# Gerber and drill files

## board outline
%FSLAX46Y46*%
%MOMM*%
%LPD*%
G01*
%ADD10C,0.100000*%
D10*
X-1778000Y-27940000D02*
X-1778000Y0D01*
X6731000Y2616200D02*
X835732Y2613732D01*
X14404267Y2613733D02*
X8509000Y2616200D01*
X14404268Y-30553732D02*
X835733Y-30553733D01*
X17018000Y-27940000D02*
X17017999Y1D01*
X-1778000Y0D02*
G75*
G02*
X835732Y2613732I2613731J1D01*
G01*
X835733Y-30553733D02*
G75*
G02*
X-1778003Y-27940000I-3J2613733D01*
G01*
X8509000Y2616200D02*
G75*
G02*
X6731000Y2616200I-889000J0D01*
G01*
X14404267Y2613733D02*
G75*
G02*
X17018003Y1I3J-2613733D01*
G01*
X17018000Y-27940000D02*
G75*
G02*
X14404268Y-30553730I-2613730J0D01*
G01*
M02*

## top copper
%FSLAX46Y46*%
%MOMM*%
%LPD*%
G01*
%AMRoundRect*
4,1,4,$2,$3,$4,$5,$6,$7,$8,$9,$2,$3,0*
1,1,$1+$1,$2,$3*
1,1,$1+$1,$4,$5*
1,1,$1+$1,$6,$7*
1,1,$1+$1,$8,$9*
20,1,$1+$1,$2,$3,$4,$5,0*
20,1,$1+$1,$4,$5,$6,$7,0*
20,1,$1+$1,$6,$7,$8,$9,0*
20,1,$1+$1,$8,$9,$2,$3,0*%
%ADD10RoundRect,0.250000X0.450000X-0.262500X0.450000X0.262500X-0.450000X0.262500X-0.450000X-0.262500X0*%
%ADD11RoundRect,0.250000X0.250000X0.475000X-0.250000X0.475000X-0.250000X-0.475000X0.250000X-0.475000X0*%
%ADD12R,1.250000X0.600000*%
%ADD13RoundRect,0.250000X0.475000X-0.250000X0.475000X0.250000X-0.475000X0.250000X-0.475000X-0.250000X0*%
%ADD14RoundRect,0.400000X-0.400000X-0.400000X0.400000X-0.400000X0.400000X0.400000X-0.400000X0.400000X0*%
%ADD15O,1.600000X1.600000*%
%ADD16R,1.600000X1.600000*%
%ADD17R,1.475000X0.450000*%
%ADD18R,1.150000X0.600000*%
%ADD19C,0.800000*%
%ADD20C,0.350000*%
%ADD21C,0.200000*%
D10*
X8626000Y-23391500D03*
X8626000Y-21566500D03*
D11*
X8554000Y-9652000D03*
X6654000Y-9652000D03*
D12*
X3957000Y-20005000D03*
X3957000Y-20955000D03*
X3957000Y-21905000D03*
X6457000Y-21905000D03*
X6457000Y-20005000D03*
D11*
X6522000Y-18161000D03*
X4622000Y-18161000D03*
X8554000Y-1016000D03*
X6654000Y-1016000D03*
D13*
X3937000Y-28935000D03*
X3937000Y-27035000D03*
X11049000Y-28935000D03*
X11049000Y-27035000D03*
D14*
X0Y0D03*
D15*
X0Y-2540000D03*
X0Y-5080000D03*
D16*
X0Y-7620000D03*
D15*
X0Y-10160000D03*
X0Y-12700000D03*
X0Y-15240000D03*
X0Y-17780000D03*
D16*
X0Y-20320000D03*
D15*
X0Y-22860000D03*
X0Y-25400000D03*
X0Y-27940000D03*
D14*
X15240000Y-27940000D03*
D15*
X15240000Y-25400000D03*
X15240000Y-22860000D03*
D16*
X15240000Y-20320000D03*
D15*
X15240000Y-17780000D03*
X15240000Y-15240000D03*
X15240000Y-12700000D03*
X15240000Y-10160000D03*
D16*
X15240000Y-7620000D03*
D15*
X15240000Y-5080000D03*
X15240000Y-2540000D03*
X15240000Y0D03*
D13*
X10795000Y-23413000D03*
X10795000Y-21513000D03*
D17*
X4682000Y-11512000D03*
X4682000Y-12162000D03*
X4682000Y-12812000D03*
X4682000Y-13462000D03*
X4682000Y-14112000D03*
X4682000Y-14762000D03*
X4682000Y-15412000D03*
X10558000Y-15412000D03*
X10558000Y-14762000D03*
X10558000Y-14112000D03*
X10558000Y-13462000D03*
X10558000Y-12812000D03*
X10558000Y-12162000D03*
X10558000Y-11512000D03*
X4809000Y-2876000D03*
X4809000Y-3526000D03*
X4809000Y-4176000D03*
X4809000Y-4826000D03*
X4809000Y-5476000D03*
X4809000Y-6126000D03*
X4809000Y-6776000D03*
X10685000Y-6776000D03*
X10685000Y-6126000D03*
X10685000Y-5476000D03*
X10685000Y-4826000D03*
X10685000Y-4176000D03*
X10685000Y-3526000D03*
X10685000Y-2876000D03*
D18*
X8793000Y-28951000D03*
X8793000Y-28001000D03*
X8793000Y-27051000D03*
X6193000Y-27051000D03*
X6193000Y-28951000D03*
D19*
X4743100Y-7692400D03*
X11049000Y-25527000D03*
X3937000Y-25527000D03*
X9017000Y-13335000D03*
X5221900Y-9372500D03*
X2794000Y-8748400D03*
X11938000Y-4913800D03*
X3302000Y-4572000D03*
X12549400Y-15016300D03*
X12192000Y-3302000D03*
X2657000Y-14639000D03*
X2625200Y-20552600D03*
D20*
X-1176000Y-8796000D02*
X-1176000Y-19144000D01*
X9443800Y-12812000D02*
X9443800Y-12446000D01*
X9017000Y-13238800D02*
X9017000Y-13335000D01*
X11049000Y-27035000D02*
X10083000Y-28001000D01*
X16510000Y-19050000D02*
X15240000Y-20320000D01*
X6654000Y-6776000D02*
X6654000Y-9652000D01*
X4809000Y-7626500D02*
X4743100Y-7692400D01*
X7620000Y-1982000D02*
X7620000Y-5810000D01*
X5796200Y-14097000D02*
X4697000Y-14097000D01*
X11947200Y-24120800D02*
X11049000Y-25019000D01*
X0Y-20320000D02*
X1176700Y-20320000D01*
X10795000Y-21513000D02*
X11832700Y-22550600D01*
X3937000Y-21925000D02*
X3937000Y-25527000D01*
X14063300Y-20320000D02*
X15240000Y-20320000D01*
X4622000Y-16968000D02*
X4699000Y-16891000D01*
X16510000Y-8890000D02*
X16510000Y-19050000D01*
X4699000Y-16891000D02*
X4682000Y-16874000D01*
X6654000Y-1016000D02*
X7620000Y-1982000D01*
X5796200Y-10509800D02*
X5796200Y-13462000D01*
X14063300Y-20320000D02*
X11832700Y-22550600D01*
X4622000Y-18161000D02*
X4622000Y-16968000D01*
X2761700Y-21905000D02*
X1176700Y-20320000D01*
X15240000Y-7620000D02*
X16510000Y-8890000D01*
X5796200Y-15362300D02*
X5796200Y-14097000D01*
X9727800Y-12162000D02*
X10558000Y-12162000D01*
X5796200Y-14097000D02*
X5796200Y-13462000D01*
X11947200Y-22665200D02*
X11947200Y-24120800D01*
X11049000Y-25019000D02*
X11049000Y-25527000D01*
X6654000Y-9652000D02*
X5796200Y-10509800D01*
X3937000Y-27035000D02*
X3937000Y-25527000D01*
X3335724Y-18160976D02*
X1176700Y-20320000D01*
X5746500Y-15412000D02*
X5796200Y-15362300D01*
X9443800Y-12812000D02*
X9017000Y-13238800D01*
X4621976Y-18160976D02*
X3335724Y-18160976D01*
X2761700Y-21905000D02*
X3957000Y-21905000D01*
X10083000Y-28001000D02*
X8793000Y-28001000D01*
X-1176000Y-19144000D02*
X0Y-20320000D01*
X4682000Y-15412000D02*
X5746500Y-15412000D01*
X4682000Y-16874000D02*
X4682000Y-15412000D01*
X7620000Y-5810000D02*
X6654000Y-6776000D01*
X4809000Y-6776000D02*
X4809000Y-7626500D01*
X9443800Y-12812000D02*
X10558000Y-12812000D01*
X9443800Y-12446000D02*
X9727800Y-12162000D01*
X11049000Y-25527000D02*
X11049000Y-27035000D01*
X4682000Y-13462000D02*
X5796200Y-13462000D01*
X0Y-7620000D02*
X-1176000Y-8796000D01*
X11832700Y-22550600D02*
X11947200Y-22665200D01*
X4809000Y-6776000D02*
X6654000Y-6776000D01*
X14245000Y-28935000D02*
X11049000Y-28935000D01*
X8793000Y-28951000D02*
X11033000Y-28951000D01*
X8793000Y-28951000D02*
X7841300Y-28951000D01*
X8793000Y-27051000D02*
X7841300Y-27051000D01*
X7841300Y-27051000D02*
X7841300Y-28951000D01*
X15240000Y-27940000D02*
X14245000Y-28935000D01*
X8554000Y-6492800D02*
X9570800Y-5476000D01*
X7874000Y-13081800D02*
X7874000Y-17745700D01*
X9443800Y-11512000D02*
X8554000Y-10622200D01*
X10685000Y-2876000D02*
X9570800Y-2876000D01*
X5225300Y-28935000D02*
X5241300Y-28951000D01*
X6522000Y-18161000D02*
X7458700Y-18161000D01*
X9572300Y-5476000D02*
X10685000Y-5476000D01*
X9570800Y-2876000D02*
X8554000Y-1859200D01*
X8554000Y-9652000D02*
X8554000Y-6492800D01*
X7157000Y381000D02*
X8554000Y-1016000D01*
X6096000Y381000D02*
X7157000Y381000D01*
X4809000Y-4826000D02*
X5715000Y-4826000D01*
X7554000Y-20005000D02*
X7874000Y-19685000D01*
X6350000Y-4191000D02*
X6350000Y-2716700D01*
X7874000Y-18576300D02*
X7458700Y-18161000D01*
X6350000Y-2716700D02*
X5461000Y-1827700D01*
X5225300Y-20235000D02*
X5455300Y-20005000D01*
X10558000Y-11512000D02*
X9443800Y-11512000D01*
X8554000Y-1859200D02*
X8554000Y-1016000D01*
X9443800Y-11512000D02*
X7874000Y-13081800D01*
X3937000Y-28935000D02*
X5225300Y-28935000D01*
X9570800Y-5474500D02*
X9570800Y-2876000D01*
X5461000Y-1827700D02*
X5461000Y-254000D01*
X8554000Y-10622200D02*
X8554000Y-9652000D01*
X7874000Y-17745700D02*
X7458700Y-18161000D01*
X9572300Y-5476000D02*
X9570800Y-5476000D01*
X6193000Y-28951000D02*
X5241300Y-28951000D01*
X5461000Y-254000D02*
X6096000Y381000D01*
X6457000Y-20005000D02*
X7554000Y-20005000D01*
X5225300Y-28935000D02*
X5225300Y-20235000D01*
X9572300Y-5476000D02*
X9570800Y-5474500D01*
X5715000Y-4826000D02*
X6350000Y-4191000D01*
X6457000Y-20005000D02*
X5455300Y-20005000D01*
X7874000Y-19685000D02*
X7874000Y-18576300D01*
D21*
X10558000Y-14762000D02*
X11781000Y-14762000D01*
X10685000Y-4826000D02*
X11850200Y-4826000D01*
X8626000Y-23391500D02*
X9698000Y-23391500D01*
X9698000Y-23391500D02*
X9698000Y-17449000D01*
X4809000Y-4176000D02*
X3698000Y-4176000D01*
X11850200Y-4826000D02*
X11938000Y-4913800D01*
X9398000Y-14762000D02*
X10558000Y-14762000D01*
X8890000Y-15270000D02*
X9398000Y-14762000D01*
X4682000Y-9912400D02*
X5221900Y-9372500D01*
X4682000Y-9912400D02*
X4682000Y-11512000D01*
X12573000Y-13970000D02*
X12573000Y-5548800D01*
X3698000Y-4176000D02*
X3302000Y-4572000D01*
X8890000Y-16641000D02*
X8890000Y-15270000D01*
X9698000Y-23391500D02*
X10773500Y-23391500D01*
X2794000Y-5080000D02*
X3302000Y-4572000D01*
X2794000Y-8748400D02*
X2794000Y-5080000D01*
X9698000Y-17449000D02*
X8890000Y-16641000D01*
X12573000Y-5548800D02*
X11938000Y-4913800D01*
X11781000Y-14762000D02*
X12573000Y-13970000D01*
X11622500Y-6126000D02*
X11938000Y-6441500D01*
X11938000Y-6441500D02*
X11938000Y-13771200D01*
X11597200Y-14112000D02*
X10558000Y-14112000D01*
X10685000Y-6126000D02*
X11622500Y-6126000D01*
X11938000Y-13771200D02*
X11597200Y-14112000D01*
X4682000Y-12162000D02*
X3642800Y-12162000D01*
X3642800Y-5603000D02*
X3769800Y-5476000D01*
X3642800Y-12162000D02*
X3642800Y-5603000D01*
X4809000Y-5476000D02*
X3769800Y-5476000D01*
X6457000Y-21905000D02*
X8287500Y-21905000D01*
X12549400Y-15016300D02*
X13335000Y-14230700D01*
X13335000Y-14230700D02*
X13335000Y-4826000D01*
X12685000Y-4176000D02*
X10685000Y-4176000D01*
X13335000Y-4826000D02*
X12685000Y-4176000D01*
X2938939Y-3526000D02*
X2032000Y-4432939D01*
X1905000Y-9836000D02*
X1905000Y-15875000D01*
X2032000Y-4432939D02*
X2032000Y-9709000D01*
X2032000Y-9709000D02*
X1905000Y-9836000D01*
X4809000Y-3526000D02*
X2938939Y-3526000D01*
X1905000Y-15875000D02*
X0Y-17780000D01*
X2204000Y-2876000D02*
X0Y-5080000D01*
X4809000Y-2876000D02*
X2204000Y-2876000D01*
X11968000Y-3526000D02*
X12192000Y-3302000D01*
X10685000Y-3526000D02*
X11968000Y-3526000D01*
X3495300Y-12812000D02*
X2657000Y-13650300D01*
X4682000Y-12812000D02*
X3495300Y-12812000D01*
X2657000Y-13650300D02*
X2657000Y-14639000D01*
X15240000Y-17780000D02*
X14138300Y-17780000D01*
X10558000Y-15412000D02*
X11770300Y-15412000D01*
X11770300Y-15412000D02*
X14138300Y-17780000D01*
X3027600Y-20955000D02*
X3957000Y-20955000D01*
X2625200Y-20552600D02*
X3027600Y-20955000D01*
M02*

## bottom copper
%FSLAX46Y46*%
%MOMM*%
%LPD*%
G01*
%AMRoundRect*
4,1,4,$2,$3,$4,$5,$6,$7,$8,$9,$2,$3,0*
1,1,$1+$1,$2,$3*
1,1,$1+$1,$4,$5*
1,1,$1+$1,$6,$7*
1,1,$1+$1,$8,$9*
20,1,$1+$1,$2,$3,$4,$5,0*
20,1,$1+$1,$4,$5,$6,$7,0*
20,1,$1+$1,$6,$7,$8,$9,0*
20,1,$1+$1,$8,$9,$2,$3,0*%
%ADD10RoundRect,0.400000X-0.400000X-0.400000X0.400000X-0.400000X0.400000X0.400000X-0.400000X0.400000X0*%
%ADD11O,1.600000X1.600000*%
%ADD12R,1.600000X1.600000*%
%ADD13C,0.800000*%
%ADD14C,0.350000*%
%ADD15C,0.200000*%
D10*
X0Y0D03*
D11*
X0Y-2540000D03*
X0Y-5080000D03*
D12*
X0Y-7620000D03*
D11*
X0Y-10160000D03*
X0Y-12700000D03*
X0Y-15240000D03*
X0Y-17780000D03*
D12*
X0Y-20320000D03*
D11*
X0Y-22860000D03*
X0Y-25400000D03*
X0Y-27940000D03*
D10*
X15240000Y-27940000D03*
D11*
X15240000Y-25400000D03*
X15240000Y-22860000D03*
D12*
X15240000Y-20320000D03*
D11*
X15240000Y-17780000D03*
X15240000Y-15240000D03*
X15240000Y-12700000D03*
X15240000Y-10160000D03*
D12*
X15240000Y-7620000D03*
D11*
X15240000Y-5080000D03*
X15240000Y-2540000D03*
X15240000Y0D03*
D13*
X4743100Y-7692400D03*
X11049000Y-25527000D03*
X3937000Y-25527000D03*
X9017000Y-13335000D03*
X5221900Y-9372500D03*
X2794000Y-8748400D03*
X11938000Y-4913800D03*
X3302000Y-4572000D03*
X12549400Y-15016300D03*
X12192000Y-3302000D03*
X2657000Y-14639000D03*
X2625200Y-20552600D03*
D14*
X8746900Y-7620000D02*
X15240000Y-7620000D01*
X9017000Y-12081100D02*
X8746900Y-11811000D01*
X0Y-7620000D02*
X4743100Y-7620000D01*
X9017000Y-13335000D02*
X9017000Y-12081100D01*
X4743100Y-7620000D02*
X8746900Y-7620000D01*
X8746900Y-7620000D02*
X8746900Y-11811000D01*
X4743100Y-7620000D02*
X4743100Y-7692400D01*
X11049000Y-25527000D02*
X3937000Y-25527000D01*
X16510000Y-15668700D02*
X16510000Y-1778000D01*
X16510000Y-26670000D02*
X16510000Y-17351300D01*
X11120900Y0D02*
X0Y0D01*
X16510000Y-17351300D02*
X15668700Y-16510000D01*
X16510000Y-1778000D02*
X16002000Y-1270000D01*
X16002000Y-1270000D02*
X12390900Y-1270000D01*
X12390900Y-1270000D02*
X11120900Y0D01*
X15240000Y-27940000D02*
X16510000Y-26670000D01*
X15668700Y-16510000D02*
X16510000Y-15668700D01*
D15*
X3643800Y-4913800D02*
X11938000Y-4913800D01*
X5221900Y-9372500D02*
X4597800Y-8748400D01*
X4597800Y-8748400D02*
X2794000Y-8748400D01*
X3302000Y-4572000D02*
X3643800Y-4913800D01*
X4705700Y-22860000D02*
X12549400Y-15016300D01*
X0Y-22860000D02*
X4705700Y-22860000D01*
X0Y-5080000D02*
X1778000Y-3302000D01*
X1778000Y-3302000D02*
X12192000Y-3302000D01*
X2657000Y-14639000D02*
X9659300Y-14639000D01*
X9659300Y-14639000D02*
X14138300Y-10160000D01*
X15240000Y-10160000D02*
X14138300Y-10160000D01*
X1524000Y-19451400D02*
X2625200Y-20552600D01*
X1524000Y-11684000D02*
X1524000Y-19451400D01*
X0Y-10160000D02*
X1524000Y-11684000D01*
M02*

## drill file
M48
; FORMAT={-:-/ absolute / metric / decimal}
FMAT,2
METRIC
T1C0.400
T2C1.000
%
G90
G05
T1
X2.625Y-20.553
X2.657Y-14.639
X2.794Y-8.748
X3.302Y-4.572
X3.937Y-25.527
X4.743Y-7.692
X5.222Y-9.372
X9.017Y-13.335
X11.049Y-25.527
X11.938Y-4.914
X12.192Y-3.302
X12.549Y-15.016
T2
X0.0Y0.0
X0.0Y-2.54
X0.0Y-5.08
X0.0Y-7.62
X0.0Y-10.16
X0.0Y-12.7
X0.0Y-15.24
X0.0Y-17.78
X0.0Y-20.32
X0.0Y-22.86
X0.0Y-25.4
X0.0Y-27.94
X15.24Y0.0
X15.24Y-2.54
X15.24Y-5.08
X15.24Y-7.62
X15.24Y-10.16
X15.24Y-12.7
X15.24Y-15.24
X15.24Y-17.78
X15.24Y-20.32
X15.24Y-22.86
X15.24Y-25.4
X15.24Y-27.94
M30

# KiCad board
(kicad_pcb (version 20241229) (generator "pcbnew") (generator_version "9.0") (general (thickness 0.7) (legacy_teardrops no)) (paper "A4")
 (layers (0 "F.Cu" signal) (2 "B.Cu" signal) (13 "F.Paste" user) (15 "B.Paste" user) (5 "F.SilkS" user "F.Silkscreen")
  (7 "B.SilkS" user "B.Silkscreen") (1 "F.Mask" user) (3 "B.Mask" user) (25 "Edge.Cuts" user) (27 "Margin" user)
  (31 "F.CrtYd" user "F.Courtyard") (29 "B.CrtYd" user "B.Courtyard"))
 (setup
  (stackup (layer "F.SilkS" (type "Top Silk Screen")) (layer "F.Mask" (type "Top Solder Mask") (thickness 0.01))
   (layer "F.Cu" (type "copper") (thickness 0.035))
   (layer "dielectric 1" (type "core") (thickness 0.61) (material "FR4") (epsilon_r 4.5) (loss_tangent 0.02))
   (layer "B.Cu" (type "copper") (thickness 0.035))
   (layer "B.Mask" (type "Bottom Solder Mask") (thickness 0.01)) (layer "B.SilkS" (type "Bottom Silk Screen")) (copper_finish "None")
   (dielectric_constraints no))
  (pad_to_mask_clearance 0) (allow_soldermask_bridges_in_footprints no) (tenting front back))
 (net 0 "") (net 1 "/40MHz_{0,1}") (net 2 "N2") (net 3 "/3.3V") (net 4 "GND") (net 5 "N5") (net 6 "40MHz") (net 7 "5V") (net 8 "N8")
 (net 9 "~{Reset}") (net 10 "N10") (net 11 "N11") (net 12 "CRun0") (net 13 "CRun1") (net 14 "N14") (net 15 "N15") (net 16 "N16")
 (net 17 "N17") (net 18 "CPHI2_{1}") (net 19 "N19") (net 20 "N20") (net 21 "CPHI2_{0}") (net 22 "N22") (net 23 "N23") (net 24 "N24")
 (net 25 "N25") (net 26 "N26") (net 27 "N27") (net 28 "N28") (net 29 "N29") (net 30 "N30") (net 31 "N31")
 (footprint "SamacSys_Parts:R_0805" (layer "F.Cu") (at 8.636 22.479)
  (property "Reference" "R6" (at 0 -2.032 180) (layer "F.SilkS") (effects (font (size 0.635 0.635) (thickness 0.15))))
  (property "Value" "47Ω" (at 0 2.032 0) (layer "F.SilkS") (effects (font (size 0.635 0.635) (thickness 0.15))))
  (pad "1" smd roundrect (at -0.01 0.9125 90) (size 1.025 1.4) (layers "F.Cu" "F.Mask" "F.Paste") (roundrect_rratio 0.243902)
   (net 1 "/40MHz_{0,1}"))
  (pad "2" smd roundrect (at -0.01 -0.9125 90) (size 1.025 1.4) (layers "F.Cu" "F.Mask" "F.Paste") (roundrect_rratio 0.243902) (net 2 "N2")))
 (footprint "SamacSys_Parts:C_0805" (layer "F.Cu") (at 7.62 9.652 90)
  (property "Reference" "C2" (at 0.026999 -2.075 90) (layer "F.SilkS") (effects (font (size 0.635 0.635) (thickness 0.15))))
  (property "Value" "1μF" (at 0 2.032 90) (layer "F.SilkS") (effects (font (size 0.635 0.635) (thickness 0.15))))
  (pad "1" smd roundrect (at 0 0.934 180) (size 1 1.45) (layers "F.Cu" "F.Mask" "F.Paste") (roundrect_rratio 0.25) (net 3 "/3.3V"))
  (pad "2" smd roundrect (at 0 -0.966 180) (size 1 1.45) (layers "F.Cu" "F.Mask" "F.Paste") (roundrect_rratio 0.25) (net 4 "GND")))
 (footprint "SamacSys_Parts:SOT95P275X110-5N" (layer "F.Cu") (at 5.207 20.955)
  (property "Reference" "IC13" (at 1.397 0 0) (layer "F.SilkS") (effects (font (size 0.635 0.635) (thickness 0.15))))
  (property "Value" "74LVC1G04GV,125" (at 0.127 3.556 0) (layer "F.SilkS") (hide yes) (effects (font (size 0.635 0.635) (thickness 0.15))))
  (pad "1" smd rect (at -1.25 -0.95 90) (size 0.6 1.25) (layers "F.Cu" "F.Mask" "F.Paste") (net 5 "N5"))
  (pad "2" smd rect (at -1.25 0 90) (size 0.6 1.25) (layers "F.Cu" "F.Mask" "F.Paste") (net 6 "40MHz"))
  (pad "3" smd rect (at -1.25 0.95 90) (size 0.6 1.25) (layers "F.Cu" "F.Mask" "F.Paste") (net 4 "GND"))
  (pad "4" smd rect (at 1.25 0.95 90) (size 0.6 1.25) (layers "F.Cu" "F.Mask" "F.Paste") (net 2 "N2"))
  (pad "5" smd rect (at 1.25 -0.95 90) (size 0.6 1.25) (layers "F.Cu" "F.Mask" "F.Paste") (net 3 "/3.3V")))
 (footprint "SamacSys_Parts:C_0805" (layer "F.Cu") (at 5.588 18.161 90)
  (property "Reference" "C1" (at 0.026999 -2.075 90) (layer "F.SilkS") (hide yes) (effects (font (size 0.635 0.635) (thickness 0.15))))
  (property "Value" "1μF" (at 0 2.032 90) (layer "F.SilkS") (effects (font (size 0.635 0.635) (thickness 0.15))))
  (pad "1" smd roundrect (at 0 0.934 180) (size 1 1.45) (layers "F.Cu" "F.Mask" "F.Paste") (roundrect_rratio 0.25) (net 3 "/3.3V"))
  (pad "2" smd roundrect (at 0 -0.966 180) (size 1 1.45) (layers "F.Cu" "F.Mask" "F.Paste") (roundrect_rratio 0.25) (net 4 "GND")))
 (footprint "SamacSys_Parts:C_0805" (layer "F.Cu") (at 7.62 1.016 90)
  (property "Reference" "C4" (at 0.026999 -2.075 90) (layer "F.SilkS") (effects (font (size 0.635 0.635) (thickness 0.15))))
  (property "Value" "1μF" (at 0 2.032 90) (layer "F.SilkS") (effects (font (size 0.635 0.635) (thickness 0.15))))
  (pad "1" smd roundrect (at 0 0.934 180) (size 1 1.45) (layers "F.Cu" "F.Mask" "F.Paste") (roundrect_rratio 0.25) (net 3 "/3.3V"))
  (pad "2" smd roundrect (at 0 -0.966 180) (size 1 1.45) (layers "F.Cu" "F.Mask" "F.Paste") (roundrect_rratio 0.25) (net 4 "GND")))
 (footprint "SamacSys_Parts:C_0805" (layer "F.Cu") (at 3.937 28.001)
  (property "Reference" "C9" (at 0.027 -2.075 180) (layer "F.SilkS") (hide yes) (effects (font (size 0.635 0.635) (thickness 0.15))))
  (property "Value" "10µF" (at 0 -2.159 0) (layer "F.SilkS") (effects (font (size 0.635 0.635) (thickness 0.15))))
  (pad "1" smd roundrect (at 0 0.934 90) (size 1 1.45) (layers "F.Cu" "F.Mask" "F.Paste") (roundrect_rratio 0.25) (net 3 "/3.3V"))
  (pad "2" smd roundrect (at 0 -0.966 90) (size 1 1.45) (layers "F.Cu" "F.Mask" "F.Paste") (roundrect_rratio 0.25) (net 4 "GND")))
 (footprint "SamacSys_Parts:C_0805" (layer "F.Cu") (at 11.049 28.001)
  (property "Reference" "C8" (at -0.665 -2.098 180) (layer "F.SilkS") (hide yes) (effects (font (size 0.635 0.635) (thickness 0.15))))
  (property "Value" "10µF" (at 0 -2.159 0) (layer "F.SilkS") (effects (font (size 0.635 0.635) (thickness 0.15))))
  (pad "1" smd roundrect (at 0 0.934 90) (size 1 1.45) (layers "F.Cu" "F.Mask" "F.Paste") (roundrect_rratio 0.25) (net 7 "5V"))
  (pad "2" smd roundrect (at 0 -0.966 90) (size 1 1.45) (layers "F.Cu" "F.Mask" "F.Paste") (roundrect_rratio 0.25) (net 4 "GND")))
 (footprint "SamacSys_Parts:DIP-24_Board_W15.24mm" (layer "F.Cu") (at 0 0)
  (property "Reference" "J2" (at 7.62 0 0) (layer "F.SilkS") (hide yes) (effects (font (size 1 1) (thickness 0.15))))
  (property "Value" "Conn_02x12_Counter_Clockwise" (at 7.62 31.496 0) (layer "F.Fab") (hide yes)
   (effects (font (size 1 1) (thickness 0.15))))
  (fp_line (start -1.778 27.94) (end -1.778 0) (stroke (width 0.1) (type solid)) (layer "Edge.Cuts"))
  (fp_line (start 6.731 -2.6162) (end 0.835732 -2.613732) (stroke (width 0.1) (type solid)) (layer "Edge.Cuts"))
  (fp_line (start 14.404267 -2.613733) (end 8.509 -2.6162) (stroke (width 0.1) (type solid)) (layer "Edge.Cuts"))
  (fp_line (start 14.404268 30.553732) (end 0.835733 30.553733) (stroke (width 0.1) (type solid)) (layer "Edge.Cuts"))
  (fp_line (start 17.018 27.94) (end 17.017999 -0.000001) (stroke (width 0.1) (type solid)) (layer "Edge.Cuts"))
  (fp_arc (start -1.778 0) (mid -1.012456 -1.848188) (end 0.835732 -2.613732) (stroke (width 0.1) (type solid)) (layer "Edge.Cuts"))
  (fp_arc (start 0.835733 30.553733) (mid -1.012456 29.788189) (end -1.778 27.94) (stroke (width 0.1) (type solid)) (layer "Edge.Cuts"))
  (fp_arc (start 8.509 -2.6162) (mid 7.62 -1.7272) (end 6.731 -2.6162) (stroke (width 0.1) (type default)) (layer "Edge.Cuts"))
  (fp_arc (start 14.404267 -2.613733) (mid 16.252455 -1.848189) (end 17.017999 -0.000001) (stroke (width 0.1) (type solid))
   (layer "Edge.Cuts"))
  (fp_arc (start 17.018 27.94) (mid 16.252455 29.788187) (end 14.404268 30.553732) (stroke (width 0.1) (type solid)) (layer "Edge.Cuts"))
  (pad "1" thru_hole roundrect (at 0 0) (size 1.6 1.6) (drill 1) (layers "*.Cu" "*.Mask") (remove_unused_layers no) (roundrect_rratio 0.25)
   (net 7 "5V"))
  (pad "2" thru_hole oval (at 0 2.54) (size 1.6 1.6) (drill 1) (layers "*.Cu" "*.Mask") (remove_unused_layers no) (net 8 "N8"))
  (pad "3" thru_hole oval (at 0 5.08) (size 1.6 1.6) (drill 1) (layers "*.Cu" "*.Mask") (remove_unused_layers no) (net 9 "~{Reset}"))
  (pad "4" thru_hole rect (at 0 7.62) (size 1.6 1.6) (drill 1) (layers "*.Cu" "*.Mask") (remove_unused_layers no) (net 4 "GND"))
  (pad "5" thru_hole oval (at 0 10.16) (size 1.6 1.6) (drill 1) (layers "*.Cu" "*.Mask") (remove_unused_layers no) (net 6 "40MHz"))
  (pad "6" thru_hole oval (at 0 12.7) (size 1.6 1.6) (drill 1) (layers "*.Cu" "*.Mask") (remove_unused_layers no) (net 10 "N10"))
  (pad "7" thru_hole oval (at 0 15.24) (size 1.6 1.6) (drill 1) (layers "*.Cu" "*.Mask") (remove_unused_layers no) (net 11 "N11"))
  (pad "8" thru_hole oval (at 0 17.78) (size 1.6 1.6) (drill 1) (layers "*.Cu" "*.Mask") (remove_unused_layers no) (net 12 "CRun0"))
  (pad "9" thru_hole rect (at 0 20.32) (size 1.6 1.6) (drill 1) (layers "*.Cu" "*.Mask") (remove_unused_layers no) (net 4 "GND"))
  (pad "10" thru_hole oval (at 0 22.86) (size 1.6 1.6) (drill 1) (layers "*.Cu" "*.Mask") (remove_unused_layers no) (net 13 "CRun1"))
  (pad "11" thru_hole oval (at 0 25.4) (size 1.6 1.6) (drill 1) (layers "*.Cu" "*.Mask") (remove_unused_layers no) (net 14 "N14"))
  (pad "12" thru_hole oval (at 0 27.94) (size 1.6 1.6) (drill 1) (layers "*.Cu" "*.Mask") (remove_unused_layers no) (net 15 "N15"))
  (pad "13" thru_hole roundrect (at 15.24 27.94) (size 1.6 1.6) (drill 1) (layers "*.Cu" "*.Mask") (remove_unused_layers no)
   (roundrect_rratio 0.25) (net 7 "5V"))
  (pad "14" thru_hole oval (at 15.24 25.4) (size 1.6 1.6) (drill 1) (layers "*.Cu" "*.Mask") (remove_unused_layers no) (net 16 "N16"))
  (pad "15" thru_hole oval (at 15.24 22.86) (size 1.6 1.6) (drill 1) (layers "*.Cu" "*.Mask") (remove_unused_layers no) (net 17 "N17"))
  (pad "16" thru_hole rect (at 15.24 20.32) (size 1.6 1.6) (drill 1) (layers "*.Cu" "*.Mask") (remove_unused_layers no) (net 4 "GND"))
  (pad "17" thru_hole oval (at 15.24 17.78 180) (size 1.6 1.6) (drill 1) (layers "*.Cu" "*.Mask") (remove_unused_layers no)
   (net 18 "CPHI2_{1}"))
  (pad "18" thru_hole oval (at 15.24 15.24 180) (size 1.6 1.6) (drill 1) (layers "*.Cu" "*.Mask") (remove_unused_layers no) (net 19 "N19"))
  (pad "19" thru_hole oval (at 15.24 12.7 180) (size 1.6 1.6) (drill 1) (layers "*.Cu" "*.Mask") (remove_unused_layers no) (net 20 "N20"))
  (pad "20" thru_hole oval (at 15.24 10.16 180) (size 1.6 1.6) (drill 1) (layers "*.Cu" "*.Mask") (remove_unused_layers no)
   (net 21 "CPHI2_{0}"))
  (pad "21" thru_hole rect (at 15.24 7.62) (size 1.6 1.6) (drill 1) (layers "*.Cu" "*.Mask") (remove_unused_layers no) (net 4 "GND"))
  (pad "22" thru_hole oval (at 15.24 5.08) (size 1.6 1.6) (drill 1) (layers "*.Cu" "*.Mask") (remove_unused_layers no) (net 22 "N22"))
  (pad "23" thru_hole oval (at 15.24 2.54) (size 1.6 1.6) (drill 1) (layers "*.Cu" "*.Mask") (remove_unused_layers no) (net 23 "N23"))
  (pad "24" thru_hole oval (at 15.24 0) (size 1.6 1.6) (drill 1) (layers "*.Cu" "*.Mask") (remove_unused_layers no) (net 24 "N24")))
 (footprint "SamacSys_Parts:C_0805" (layer "F.Cu") (at 10.795 22.479)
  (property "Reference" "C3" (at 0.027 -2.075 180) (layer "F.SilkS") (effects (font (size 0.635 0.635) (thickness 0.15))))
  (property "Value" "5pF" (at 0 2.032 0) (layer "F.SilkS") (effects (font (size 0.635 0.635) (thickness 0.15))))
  (pad "1" smd roundrect (at 0 0.934 90) (size 1 1.45) (layers "F.Cu" "F.Mask" "F.Paste") (roundrect_rratio 0.25) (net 1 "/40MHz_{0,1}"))
  (pad "2" smd roundrect (at 0 -0.966 90) (size 1 1.45) (layers "F.Cu" "F.Mask" "F.Paste") (roundrect_rratio 0.25) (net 4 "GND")))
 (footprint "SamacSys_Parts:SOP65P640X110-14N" (layer "F.Cu") (at 7.62 13.462)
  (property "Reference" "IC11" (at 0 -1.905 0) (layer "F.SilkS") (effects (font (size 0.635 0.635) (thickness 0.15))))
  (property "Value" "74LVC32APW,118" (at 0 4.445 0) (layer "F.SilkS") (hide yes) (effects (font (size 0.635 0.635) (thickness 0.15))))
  (pad "1" smd rect (at -2.938 -1.95 90) (size 0.45 1.475) (layers "F.Cu" "F.Mask" "F.Paste") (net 1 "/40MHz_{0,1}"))
  (pad "2" smd rect (at -2.938 -1.3 90) (size 0.45 1.475) (layers "F.Cu" "F.Mask" "F.Paste") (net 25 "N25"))
  (pad "3" smd rect (at -2.938 -0.65 90) (size 0.45 1.475) (layers "F.Cu" "F.Mask" "F.Paste") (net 21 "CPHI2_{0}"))
  (pad "4" smd rect (at -2.938 0 90) (size 0.45 1.475) (layers "F.Cu" "F.Mask" "F.Paste") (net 4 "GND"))
  (pad "5" smd rect (at -2.938 0.65 90) (size 0.45 1.475) (layers "F.Cu" "F.Mask" "F.Paste") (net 4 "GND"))
  (pad "6" smd rect (at -2.938 1.3 90) (size 0.45 1.475) (layers "F.Cu" "F.Mask" "F.Paste") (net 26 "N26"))
  (pad "7" smd rect (at -2.938 1.95 90) (size 0.45 1.475) (layers "F.Cu" "F.Mask" "F.Paste") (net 4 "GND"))
  (pad "8" smd rect (at 2.938 1.95 90) (size 0.45 1.475) (layers "F.Cu" "F.Mask" "F.Paste") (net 18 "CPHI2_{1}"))
  (pad "9" smd rect (at 2.938 1.3 90) (size 0.45 1.475) (layers "F.Cu" "F.Mask" "F.Paste") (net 1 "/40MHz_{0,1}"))
  (pad "10" smd rect (at 2.938 0.65 90) (size 0.45 1.475) (layers "F.Cu" "F.Mask" "F.Paste") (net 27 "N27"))
  (pad "11" smd rect (at 2.938 0 90) (size 0.45 1.475) (layers "F.Cu" "F.Mask" "F.Paste") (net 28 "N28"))
  (pad "12" smd rect (at 2.938 -0.65 90) (size 0.45 1.475) (layers "F.Cu" "F.Mask" "F.Paste") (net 4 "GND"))
  (pad "13" smd rect (at 2.938 -1.3 90) (size 0.45 1.475) (layers "F.Cu" "F.Mask" "F.Paste") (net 4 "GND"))
  (pad "14" smd rect (at 2.938 -1.95 90) (size 0.45 1.475) (layers "F.Cu" "F.Mask" "F.Paste") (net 3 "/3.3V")))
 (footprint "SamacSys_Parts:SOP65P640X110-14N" (layer "F.Cu") (at 7.747 4.826)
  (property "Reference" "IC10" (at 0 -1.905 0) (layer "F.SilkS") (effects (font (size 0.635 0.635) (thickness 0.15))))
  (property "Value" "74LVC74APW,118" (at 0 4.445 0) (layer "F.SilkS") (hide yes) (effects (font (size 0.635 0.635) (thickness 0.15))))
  (pad "1" smd rect (at -2.938 -1.95 90) (size 0.45 1.475) (layers "F.Cu" "F.Mask" "F.Paste") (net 9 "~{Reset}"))
  (pad "2" smd rect (at -2.938 -1.3 90) (size 0.45 1.475) (layers "F.Cu" "F.Mask" "F.Paste") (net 12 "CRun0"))
  (pad "3" smd rect (at -2.938 -0.65 90) (size 0.45 1.475) (layers "F.Cu" "F.Mask" "F.Paste") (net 1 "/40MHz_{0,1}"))
  (pad "4" smd rect (at -2.938 0 90) (size 0.45 1.475) (layers "F.Cu" "F.Mask" "F.Paste") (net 3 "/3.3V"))
  (pad "5" smd rect (at -2.938 0.65 90) (size 0.45 1.475) (layers "F.Cu" "F.Mask" "F.Paste") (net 25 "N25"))
  (pad "6" smd rect (at -2.938 1.3 90) (size 0.45 1.475) (layers "F.Cu" "F.Mask" "F.Paste") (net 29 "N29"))
  (pad "7" smd rect (at -2.938 1.95 90) (size 0.45 1.475) (layers "F.Cu" "F.Mask" "F.Paste") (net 4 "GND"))
  (pad "8" smd rect (at 2.938 1.95 90) (size 0.45 1.475) (layers "F.Cu" "F.Mask" "F.Paste") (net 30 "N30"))
  (pad "9" smd rect (at 2.938 1.3 90) (size 0.45 1.475) (layers "F.Cu" "F.Mask" "F.Paste") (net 27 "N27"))
  (pad "10" smd rect (at 2.938 0.65 90) (size 0.45 1.475) (layers "F.Cu" "F.Mask" "F.Paste") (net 3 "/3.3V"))
  (pad "11" smd rect (at 2.938 0 90) (size 0.45 1.475) (layers "F.Cu" "F.Mask" "F.Paste") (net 1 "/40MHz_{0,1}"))
  (pad "12" smd rect (at 2.938 -0.65 90) (size 0.45 1.475) (layers "F.Cu" "F.Mask" "F.Paste") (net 13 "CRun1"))
  (pad "13" smd rect (at 2.938 -1.3 90) (size 0.45 1.475) (layers "F.Cu" "F.Mask" "F.Paste") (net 9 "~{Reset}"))
  (pad "14" smd rect (at 2.938 -1.95 90) (size 0.45 1.475) (layers "F.Cu" "F.Mask" "F.Paste") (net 3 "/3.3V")))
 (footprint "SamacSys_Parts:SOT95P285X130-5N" (layer "F.Cu") (at 7.493 28.001 180)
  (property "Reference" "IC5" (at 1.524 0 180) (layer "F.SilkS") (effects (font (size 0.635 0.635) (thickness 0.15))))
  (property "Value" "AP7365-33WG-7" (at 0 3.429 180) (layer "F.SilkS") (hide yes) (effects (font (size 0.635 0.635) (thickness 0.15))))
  (pad "1" smd rect (at -1.3 -0.95 270) (size 0.6 1.15) (layers "F.Cu" "F.Mask" "F.Paste") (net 7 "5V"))
  (pad "2" smd rect (at -1.3 0 270) (size 0.6 1.15) (layers "F.Cu" "F.Mask" "F.Paste") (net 4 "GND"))
  (pad "3" smd rect (at -1.3 0.95 270) (size 0.6 1.15) (layers "F.Cu" "F.Mask" "F.Paste") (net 7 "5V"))
  (pad "4" smd rect (at 1.3 0.95 270) (size 0.6 1.15) (layers "F.Cu" "F.Mask" "F.Paste") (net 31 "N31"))
  (pad "5" smd rect (at 1.3 -0.95 270) (size 0.6 1.15) (layers "F.Cu" "F.Mask" "F.Paste") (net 3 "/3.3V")))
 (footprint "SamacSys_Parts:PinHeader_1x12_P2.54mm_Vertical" (layer "B.Cu") (at 0 0 180)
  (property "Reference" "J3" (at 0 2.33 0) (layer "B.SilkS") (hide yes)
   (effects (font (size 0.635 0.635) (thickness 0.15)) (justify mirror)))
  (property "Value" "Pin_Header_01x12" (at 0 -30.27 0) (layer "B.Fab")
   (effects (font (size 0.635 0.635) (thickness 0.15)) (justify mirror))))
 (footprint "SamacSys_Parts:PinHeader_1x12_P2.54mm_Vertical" (layer "B.Cu") (at 15.24 0 180)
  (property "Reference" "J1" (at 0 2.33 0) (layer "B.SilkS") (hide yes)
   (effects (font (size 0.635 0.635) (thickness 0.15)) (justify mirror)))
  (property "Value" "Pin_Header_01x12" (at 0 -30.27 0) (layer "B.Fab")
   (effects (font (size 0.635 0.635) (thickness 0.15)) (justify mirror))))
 (segment (start -1.176 8.796) (end -1.176 19.144) (width 0.35) (layer "F.Cu") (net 4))
 (segment (start 9.4438 12.812) (end 9.4438 12.446) (width 0.35) (layer "F.Cu") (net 4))
 (segment (start 9.017 13.2388) (end 9.017 13.335) (width 0.35) (layer "F.Cu") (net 4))
 (segment (start 11.049 27.035) (end 10.083 28.001) (width 0.35) (layer "F.Cu") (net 4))
 (segment (start 16.51 19.05) (end 15.24 20.32) (width 0.35) (layer "F.Cu") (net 4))
 (segment (start 6.654 6.776) (end 6.654 9.652) (width 0.35) (layer "F.Cu") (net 4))
 (segment (start 4.809 7.6265) (end 4.7431 7.6924) (width 0.35) (layer "F.Cu") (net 4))
 (segment (start 7.62 1.982) (end 7.62 5.81) (width 0.35) (layer "F.Cu") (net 4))
 (segment (start 5.7962 14.097) (end 4.697 14.097) (width 0.35) (layer "F.Cu") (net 4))
 (segment (start 11.9472 24.1208) (end 11.049 25.019) (width 0.35) (layer "F.Cu") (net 4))
 (segment (start 0 20.32) (end 1.1767 20.32) (width 0.35) (layer "F.Cu") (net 4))
 (segment (start 10.795 21.513) (end 11.8327 22.5506) (width 0.35) (layer "F.Cu") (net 4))
 (segment (start 3.937 21.925) (end 3.937 25.527) (width 0.35) (layer "F.Cu") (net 4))
 (segment (start 14.0633 20.32) (end 15.24 20.32) (width 0.35) (layer "F.Cu") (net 4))
 (segment (start 4.622 16.968) (end 4.699 16.891) (width 0.35) (layer "F.Cu") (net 4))
 (segment (start 16.51 8.89) (end 16.51 19.05) (width 0.35) (layer "F.Cu") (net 4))
 (segment (start 4.699 16.891) (end 4.682 16.874) (width 0.35) (layer "F.Cu") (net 4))
 (segment (start 6.654 1.016) (end 7.62 1.982) (width 0.35) (layer "F.Cu") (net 4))
 (segment (start 5.7962 10.5098) (end 5.7962 13.462) (width 0.35) (layer "F.Cu") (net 4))
 (segment (start 14.0633 20.32) (end 11.8327 22.5506) (width 0.35) (layer "F.Cu") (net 4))
 (segment (start 4.622 18.161) (end 4.622 16.968) (width 0.35) (layer "F.Cu") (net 4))
 (segment (start 2.7617 21.905) (end 1.1767 20.32) (width 0.35) (layer "F.Cu") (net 4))
 (segment (start 15.24 7.62) (end 16.51 8.89) (width 0.35) (layer "F.Cu") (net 4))
 (segment (start 5.7962 15.3623) (end 5.7962 14.097) (width 0.35) (layer "F.Cu") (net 4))
 (segment (start 9.7278 12.162) (end 10.558 12.162) (width 0.35) (layer "F.Cu") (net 4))
 (segment (start 5.7962 14.097) (end 5.7962 13.462) (width 0.35) (layer "F.Cu") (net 4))
 (segment (start 11.9472 22.6652) (end 11.9472 24.1208) (width 0.35) (layer "F.Cu") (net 4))
 (segment (start 11.049 25.019) (end 11.049 25.527) (width 0.35) (layer "F.Cu") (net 4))
 (segment (start 6.654 9.652) (end 5.7962 10.5098) (width 0.35) (layer "F.Cu") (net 4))
 (segment (start 3.937 27.035) (end 3.937 25.527) (width 0.35) (layer "F.Cu") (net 4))
 (segment (start 3.335724 18.160976) (end 1.1767 20.32) (width 0.35) (layer "F.Cu") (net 4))
 (segment (start 5.7465 15.412) (end 5.7962 15.3623) (width 0.35) (layer "F.Cu") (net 4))
 (segment (start 9.4438 12.812) (end 9.017 13.2388) (width 0.35) (layer "F.Cu") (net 4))
 (segment (start 4.621976 18.160976) (end 3.335724 18.160976) (width 0.35) (layer "F.Cu") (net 4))
 (segment (start 2.7617 21.905) (end 3.957 21.905) (width 0.35) (layer "F.Cu") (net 4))
 (segment (start 10.083 28.001) (end 8.793 28.001) (width 0.35) (layer "F.Cu") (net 4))
 (segment (start -1.176 19.144) (end 0 20.32) (width 0.35) (layer "F.Cu") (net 4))
 (segment (start 4.682 15.412) (end 5.7465 15.412) (width 0.35) (layer "F.Cu") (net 4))
 (segment (start 4.682 16.874) (end 4.682 15.412) (width 0.35) (layer "F.Cu") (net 4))
 (segment (start 7.62 5.81) (end 6.654 6.776) (width 0.35) (layer "F.Cu") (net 4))
 (segment (start 4.809 6.776) (end 4.809 7.6265) (width 0.35) (layer "F.Cu") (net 4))
 (segment (start 9.4438 12.812) (end 10.558 12.812) (width 0.35) (layer "F.Cu") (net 4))
 (segment (start 9.4438 12.446) (end 9.7278 12.162) (width 0.35) (layer "F.Cu") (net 4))
 (segment (start 11.049 25.527) (end 11.049 27.035) (width 0.35) (layer "F.Cu") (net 4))
 (segment (start 4.682 13.462) (end 5.7962 13.462) (width 0.35) (layer "F.Cu") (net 4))
 (segment (start 0 7.62) (end -1.176 8.796) (width 0.35) (layer "F.Cu") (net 4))
 (segment (start 11.8327 22.5506) (end 11.9472 22.6652) (width 0.35) (layer "F.Cu") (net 4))
 (segment (start 4.809 6.776) (end 6.654 6.776) (width 0.35) (layer "F.Cu") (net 4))
 (via (at 4.7431 7.6924) (size 0.8) (drill 0.4) (layers "F.Cu" "B.Cu") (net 4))
 (via (at 11.049 25.527) (size 0.8) (drill 0.4) (layers "F.Cu" "B.Cu") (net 4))
 (via (at 3.937 25.527) (size 0.8) (drill 0.4) (layers "F.Cu" "B.Cu") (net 4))
 (via (at 9.017 13.335) (size 0.8) (drill 0.4) (layers "F.Cu" "B.Cu") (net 4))
 (segment (start 8.7469 7.62) (end 15.24 7.62) (width 0.35) (layer "B.Cu") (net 4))
 (segment (start 9.017 12.0811) (end 8.7469 11.811) (width 0.35) (layer "B.Cu") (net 4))
 (segment (start 0 7.62) (end 4.7431 7.62) (width 0.35) (layer "B.Cu") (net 4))
 (segment (start 9.017 13.335) (end 9.017 12.0811) (width 0.35) (layer "B.Cu") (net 4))
 (segment (start 4.7431 7.62) (end 8.7469 7.62) (width 0.35) (layer "B.Cu") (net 4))
 (segment (start 8.7469 7.62) (end 8.7469 11.811) (width 0.35) (layer "B.Cu") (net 4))
 (segment (start 4.7431 7.62) (end 4.7431 7.6924) (width 0.35) (layer "B.Cu") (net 4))
 (segment (start 11.049 25.527) (end 3.937 25.527) (width 0.35) (layer "B.Cu") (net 4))
 (segment (start 14.245 28.935) (end 11.049 28.935) (width 0.35) (layer "F.Cu") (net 7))
 (segment (start 8.793 28.951) (end 11.033 28.951) (width 0.35) (layer "F.Cu") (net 7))
 (segment (start 8.793 28.951) (end 7.8413 28.951) (width 0.35) (layer "F.Cu") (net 7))
 (segment (start 8.793 27.051) (end 7.8413 27.051) (width 0.35) (layer "F.Cu") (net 7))
 (segment (start 7.8413 27.051) (end 7.8413 28.951) (width 0.35) (layer "F.Cu") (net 7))
 (segment (start 15.24 27.94) (end 14.245 28.935) (width 0.35) (layer "F.Cu") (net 7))
 (segment (start 16.51 15.6687) (end 16.51 1.778) (width 0.35) (layer "B.Cu") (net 7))
 (segment (start 16.51 26.67) (end 16.51 17.3513) (width 0.35) (layer "B.Cu") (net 7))
 (segment (start 11.1209 0) (end 0 0) (width 0.35) (layer "B.Cu") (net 7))
 (segment (start 16.51 17.3513) (end 15.6687 16.51) (width 0.35) (layer "B.Cu") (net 7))
 (segment (start 16.51 1.778) (end 16.002 1.27) (width 0.35) (layer "B.Cu") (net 7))
 (segment (start 16.002 1.27) (end 12.3909 1.27) (width 0.35) (layer "B.Cu") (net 7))
 (segment (start 12.3909 1.27) (end 11.1209 0) (width 0.35) (layer "B.Cu") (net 7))
 (segment (start 15.24 27.94) (end 16.51 26.67) (width 0.35) (layer "B.Cu") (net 7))
 (segment (start 15.6687 16.51) (end 16.51 15.6687) (width 0.35) (layer "B.Cu") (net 7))
 (segment (start 8.554 6.4928) (end 9.5708 5.476) (width 0.35) (layer "F.Cu") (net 3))
 (segment (start 7.874 13.0818) (end 7.874 17.7457) (width 0.35) (layer "F.Cu") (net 3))
 (segment (start 9.4438 11.512) (end 8.554 10.6222) (width 0.35) (layer "F.Cu") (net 3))
 (segment (start 10.685 2.876) (end 9.5708 2.876) (width 0.35) (layer "F.Cu") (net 3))
 (segment (start 5.2253 28.935) (end 5.2413 28.951) (width 0.35) (layer "F.Cu") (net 3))
 (segment (start 6.522 18.161) (end 7.4587 18.161) (width 0.35) (layer "F.Cu") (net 3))
 (segment (start 9.5723 5.476) (end 10.685 5.476) (width 0.35) (layer "F.Cu") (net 3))
 (segment (start 9.5708 2.876) (end 8.554 1.8592) (width 0.35) (layer "F.Cu") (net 3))
 (segment (start 8.554 9.652) (end 8.554 6.4928) (width 0.35) (layer "F.Cu") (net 3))
 (segment (start 7.157 -0.381) (end 8.554 1.016) (width 0.35) (layer "F.Cu") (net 3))
 (segment (start 6.096 -0.381) (end 7.157 -0.381) (width 0.35) (layer "F.Cu") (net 3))
 (segment (start 4.809 4.826) (end 5.715 4.826) (width 0.35) (layer "F.Cu") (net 3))
 (segment (start 7.554 20.005) (end 7.874 19.685) (width 0.35) (layer "F.Cu") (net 3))
 (segment (start 6.35 4.191) (end 6.35 2.7167) (width 0.35) (layer "F.Cu") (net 3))
 (segment (start 7.874 18.5763) (end 7.4587 18.161) (width 0.35) (layer "F.Cu") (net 3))
 (segment (start 6.35 2.7167) (end 5.461 1.8277) (width 0.35) (layer "F.Cu") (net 3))
 (segment (start 5.2253 20.235) (end 5.4553 20.005) (width 0.35) (layer "F.Cu") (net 3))
 (segment (start 10.558 11.512) (end 9.4438 11.512) (width 0.35) (layer "F.Cu") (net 3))
 (segment (start 8.554 1.8592) (end 8.554 1.016) (width 0.35) (layer "F.Cu") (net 3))
 (segment (start 9.4438 11.512) (end 7.874 13.0818) (width 0.35) (layer "F.Cu") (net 3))
 (segment (start 3.937 28.935) (end 5.2253 28.935) (width 0.35) (layer "F.Cu") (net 3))
 (segment (start 9.5708 5.4745) (end 9.5708 2.876) (width 0.35) (layer "F.Cu") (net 3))
 (segment (start 5.461 1.8277) (end 5.461 0.254) (width 0.35) (layer "F.Cu") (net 3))
 (segment (start 8.554 10.6222) (end 8.554 9.652) (width 0.35) (layer "F.Cu") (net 3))
 (segment (start 7.874 17.7457) (end 7.4587 18.161) (width 0.35) (layer "F.Cu") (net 3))
 (segment (start 9.5723 5.476) (end 9.5708 5.476) (width 0.35) (layer "F.Cu") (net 3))
 (segment (start 6.193 28.951) (end 5.2413 28.951) (width 0.35) (layer "F.Cu") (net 3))
 (segment (start 5.461 0.254) (end 6.096 -0.381) (width 0.35) (layer "F.Cu") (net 3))
 (segment (start 6.457 20.005) (end 7.554 20.005) (width 0.35) (layer "F.Cu") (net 3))
 (segment (start 5.2253 28.935) (end 5.2253 20.235) (width 0.35) (layer "F.Cu") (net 3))
 (segment (start 9.5723 5.476) (end 9.5708 5.4745) (width 0.35) (layer "F.Cu") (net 3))
 (segment (start 5.715 4.826) (end 6.35 4.191) (width 0.35) (layer "F.Cu") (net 3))
 (segment (start 6.457 20.005) (end 5.4553 20.005) (width 0.35) (layer "F.Cu") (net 3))
 (segment (start 7.874 19.685) (end 7.874 18.5763) (width 0.35) (layer "F.Cu") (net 3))
 (segment (start 10.558 14.762) (end 11.781 14.762) (width 0.2) (layer "F.Cu") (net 1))
 (segment (start 10.685 4.826) (end 11.8502 4.826) (width 0.2) (layer "F.Cu") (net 1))
 (segment (start 8.626 23.3915) (end 9.698 23.3915) (width 0.2) (layer "F.Cu") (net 1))
 (segment (start 9.698 23.3915) (end 9.698 17.449) (width 0.2) (layer "F.Cu") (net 1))
 (segment (start 4.809 4.176) (end 3.698 4.176) (width 0.2) (layer "F.Cu") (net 1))
 (segment (start 11.8502 4.826) (end 11.938 4.9138) (width 0.2) (layer "F.Cu") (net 1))
 (segment (start 9.398 14.762) (end 10.558 14.762) (width 0.2) (layer "F.Cu") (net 1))
 (segment (start 8.89 15.27) (end 9.398 14.762) (width 0.2) (layer "F.Cu") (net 1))
 (segment (start 4.682 9.9124) (end 5.2219 9.3725) (width 0.2) (layer "F.Cu") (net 1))
 (segment (start 4.682 9.9124) (end 4.682 11.512) (width 0.2) (layer "F.Cu") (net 1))
 (segment (start 12.573 13.97) (end 12.573 5.5488) (width 0.2) (layer "F.Cu") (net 1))
 (segment (start 3.698 4.176) (end 3.302 4.572) (width 0.2) (layer "F.Cu") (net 1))
 (segment (start 8.89 16.641) (end 8.89 15.27) (width 0.2) (layer "F.Cu") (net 1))
 (segment (start 9.698 23.3915) (end 10.7735 23.3915) (width 0.2) (layer "F.Cu") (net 1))
 (segment (start 2.794 5.08) (end 3.302 4.572) (width 0.2) (layer "F.Cu") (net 1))
 (segment (start 2.794 8.7484) (end 2.794 5.08) (width 0.2) (layer "F.Cu") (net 1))
 (segment (start 9.698 17.449) (end 8.89 16.641) (width 0.2) (layer "F.Cu") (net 1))
 (segment (start 12.573 5.5488) (end 11.938 4.9138) (width 0.2) (layer "F.Cu") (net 1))
 (segment (start 11.781 14.762) (end 12.573 13.97) (width 0.2) (layer "F.Cu") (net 1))
 (via (at 5.2219 9.3725) (size 0.8) (drill 0.4) (layers "F.Cu" "B.Cu") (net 1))
 (via (at 2.794 8.7484) (size 0.8) (drill 0.4) (layers "F.Cu" "B.Cu") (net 1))
 (via (at 11.938 4.9138) (size 0.8) (drill 0.4) (layers "F.Cu" "B.Cu") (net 1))
 (via (at 3.302 4.572) (size 0.8) (drill 0.4) (layers "F.Cu" "B.Cu") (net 1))
 (segment (start 3.6438 4.9138) (end 11.938 4.9138) (width 0.2) (layer "B.Cu") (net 1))
 (segment (start 5.2219 9.3725) (end 4.5978 8.7484) (width 0.2) (layer "B.Cu") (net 1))
 (segment (start 4.5978 8.7484) (end 2.794 8.7484) (width 0.2) (layer "B.Cu") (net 1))
 (segment (start 3.302 4.572) (end 3.6438 4.9138) (width 0.2) (layer "B.Cu") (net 1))
 (segment (start 11.6225 6.126) (end 11.938 6.4415) (width 0.2) (layer "F.Cu") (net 27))
 (segment (start 11.938 6.4415) (end 11.938 13.7712) (width 0.2) (layer "F.Cu") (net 27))
 (segment (start 11.5972 14.112) (end 10.558 14.112) (width 0.2) (layer "F.Cu") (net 27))
 (segment (start 10.685 6.126) (end 11.6225 6.126) (width 0.2) (layer "F.Cu") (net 27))
 (segment (start 11.938 13.7712) (end 11.5972 14.112) (width 0.2) (layer "F.Cu") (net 27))
 (segment (start 4.682 12.162) (end 3.6428 12.162) (width 0.2) (layer "F.Cu") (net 25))
 (segment (start 3.6428 5.603) (end 3.7698 5.476) (width 0.2) (layer "F.Cu") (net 25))
 (segment (start 3.6428 12.162) (end 3.6428 5.603) (width 0.2) (layer "F.Cu") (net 25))
 (segment (start 4.809 5.476) (end 3.7698 5.476) (width 0.2) (layer "F.Cu") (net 25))
 (segment (start 6.457 21.905) (end 8.2875 21.905) (width 0.2) (layer "F.Cu") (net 2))
 (segment (start 12.5494 15.0163) (end 13.335 14.2307) (width 0.2) (layer "F.Cu") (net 13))
 (segment (start 13.335 14.2307) (end 13.335 4.826) (width 0.2) (layer "F.Cu") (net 13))
 (segment (start 12.685 4.176) (end 10.685 4.176) (width 0.2) (layer "F.Cu") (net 13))
 (segment (start 13.335 4.826) (end 12.685 4.176) (width 0.2) (layer "F.Cu") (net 13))
 (via (at 12.5494 15.0163) (size 0.8) (drill 0.4) (layers "F.Cu" "B.Cu") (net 13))
 (segment (start 4.7057 22.86) (end 12.5494 15.0163) (width 0.2) (layer "B.Cu") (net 13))
 (segment (start 0 22.86) (end 4.7057 22.86) (width 0.2) (layer "B.Cu") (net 13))
 (segment (start 2.938939 3.526) (end 2.032 4.432939) (width 0.2) (layer "F.Cu") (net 12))
 (segment (start 1.905 9.836) (end 1.905 15.875) (width 0.2) (layer "F.Cu") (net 12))
 (segment (start 2.032 4.432939) (end 2.032 9.709) (width 0.2) (layer "F.Cu") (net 12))
 (segment (start 2.032 9.709) (end 1.905 9.836) (width 0.2) (layer "F.Cu") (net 12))
 (segment (start 4.809 3.526) (end 2.938939 3.526) (width 0.2) (layer "F.Cu") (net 12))
 (segment (start 1.905 15.875) (end 0 17.78) (width 0.2) (layer "F.Cu") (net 12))
 (segment (start 2.204 2.876) (end 0 5.08) (width 0.2) (layer "F.Cu") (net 9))
 (segment (start 4.809 2.876) (end 2.204 2.876) (width 0.2) (layer "F.Cu") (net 9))
 (segment (start 11.968 3.526) (end 12.192 3.302) (width 0.2) (layer "F.Cu") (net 9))
 (segment (start 10.685 3.526) (end 11.968 3.526) (width 0.2) (layer "F.Cu") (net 9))
 (via (at 12.192 3.302) (size 0.8) (drill 0.4) (layers "F.Cu" "B.Cu") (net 9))
 (segment (start 0 5.08) (end 1.778 3.302) (width 0.2) (layer "B.Cu") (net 9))
 (segment (start 1.778 3.302) (end 12.192 3.302) (width 0.2) (layer "B.Cu") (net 9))
 (segment (start 3.4953 12.812) (end 2.657 13.6503) (width 0.2) (layer "F.Cu") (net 21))
 (segment (start 4.682 12.812) (end 3.4953 12.812) (width 0.2) (layer "F.Cu") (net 21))
 (segment (start 2.657 13.6503) (end 2.657 14.639) (width 0.2) (layer "F.Cu") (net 21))
 (via (at 2.657 14.639) (size 0.8) (drill 0.4) (layers "F.Cu" "B.Cu") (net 21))
 (segment (start 2.657 14.639) (end 9.6593 14.639) (width 0.2) (layer "B.Cu") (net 21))
 (segment (start 9.6593 14.639) (end 14.1383 10.16) (width 0.2) (layer "B.Cu") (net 21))
 (segment (start 15.24 10.16) (end 14.1383 10.16) (width 0.2) (layer "B.Cu") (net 21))
 (segment (start 15.24 17.78) (end 14.1383 17.78) (width 0.2) (layer "F.Cu") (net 18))
 (segment (start 10.558 15.412) (end 11.7703 15.412) (width 0.2) (layer "F.Cu") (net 18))
 (segment (start 11.7703 15.412) (end 14.1383 17.78) (width 0.2) (layer "F.Cu") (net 18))
 (segment (start 3.0276 20.955) (end 3.957 20.955) (width 0.2) (layer "F.Cu") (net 6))
 (segment (start 2.6252 20.5526) (end 3.0276 20.955) (width 0.2) (layer "F.Cu") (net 6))
 (via (at 2.6252 20.5526) (size 0.8) (drill 0.4) (layers "F.Cu" "B.Cu") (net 6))
 (segment (start 1.524 19.4514) (end 2.6252 20.5526) (width 0.2) (layer "B.Cu") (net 6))
 (segment (start 1.524 11.684) (end 1.524 19.4514) (width 0.2) (layer "B.Cu") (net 6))
 (segment (start 0 10.16) (end 1.524 11.684) (width 0.2) (layer "B.Cu") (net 6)))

